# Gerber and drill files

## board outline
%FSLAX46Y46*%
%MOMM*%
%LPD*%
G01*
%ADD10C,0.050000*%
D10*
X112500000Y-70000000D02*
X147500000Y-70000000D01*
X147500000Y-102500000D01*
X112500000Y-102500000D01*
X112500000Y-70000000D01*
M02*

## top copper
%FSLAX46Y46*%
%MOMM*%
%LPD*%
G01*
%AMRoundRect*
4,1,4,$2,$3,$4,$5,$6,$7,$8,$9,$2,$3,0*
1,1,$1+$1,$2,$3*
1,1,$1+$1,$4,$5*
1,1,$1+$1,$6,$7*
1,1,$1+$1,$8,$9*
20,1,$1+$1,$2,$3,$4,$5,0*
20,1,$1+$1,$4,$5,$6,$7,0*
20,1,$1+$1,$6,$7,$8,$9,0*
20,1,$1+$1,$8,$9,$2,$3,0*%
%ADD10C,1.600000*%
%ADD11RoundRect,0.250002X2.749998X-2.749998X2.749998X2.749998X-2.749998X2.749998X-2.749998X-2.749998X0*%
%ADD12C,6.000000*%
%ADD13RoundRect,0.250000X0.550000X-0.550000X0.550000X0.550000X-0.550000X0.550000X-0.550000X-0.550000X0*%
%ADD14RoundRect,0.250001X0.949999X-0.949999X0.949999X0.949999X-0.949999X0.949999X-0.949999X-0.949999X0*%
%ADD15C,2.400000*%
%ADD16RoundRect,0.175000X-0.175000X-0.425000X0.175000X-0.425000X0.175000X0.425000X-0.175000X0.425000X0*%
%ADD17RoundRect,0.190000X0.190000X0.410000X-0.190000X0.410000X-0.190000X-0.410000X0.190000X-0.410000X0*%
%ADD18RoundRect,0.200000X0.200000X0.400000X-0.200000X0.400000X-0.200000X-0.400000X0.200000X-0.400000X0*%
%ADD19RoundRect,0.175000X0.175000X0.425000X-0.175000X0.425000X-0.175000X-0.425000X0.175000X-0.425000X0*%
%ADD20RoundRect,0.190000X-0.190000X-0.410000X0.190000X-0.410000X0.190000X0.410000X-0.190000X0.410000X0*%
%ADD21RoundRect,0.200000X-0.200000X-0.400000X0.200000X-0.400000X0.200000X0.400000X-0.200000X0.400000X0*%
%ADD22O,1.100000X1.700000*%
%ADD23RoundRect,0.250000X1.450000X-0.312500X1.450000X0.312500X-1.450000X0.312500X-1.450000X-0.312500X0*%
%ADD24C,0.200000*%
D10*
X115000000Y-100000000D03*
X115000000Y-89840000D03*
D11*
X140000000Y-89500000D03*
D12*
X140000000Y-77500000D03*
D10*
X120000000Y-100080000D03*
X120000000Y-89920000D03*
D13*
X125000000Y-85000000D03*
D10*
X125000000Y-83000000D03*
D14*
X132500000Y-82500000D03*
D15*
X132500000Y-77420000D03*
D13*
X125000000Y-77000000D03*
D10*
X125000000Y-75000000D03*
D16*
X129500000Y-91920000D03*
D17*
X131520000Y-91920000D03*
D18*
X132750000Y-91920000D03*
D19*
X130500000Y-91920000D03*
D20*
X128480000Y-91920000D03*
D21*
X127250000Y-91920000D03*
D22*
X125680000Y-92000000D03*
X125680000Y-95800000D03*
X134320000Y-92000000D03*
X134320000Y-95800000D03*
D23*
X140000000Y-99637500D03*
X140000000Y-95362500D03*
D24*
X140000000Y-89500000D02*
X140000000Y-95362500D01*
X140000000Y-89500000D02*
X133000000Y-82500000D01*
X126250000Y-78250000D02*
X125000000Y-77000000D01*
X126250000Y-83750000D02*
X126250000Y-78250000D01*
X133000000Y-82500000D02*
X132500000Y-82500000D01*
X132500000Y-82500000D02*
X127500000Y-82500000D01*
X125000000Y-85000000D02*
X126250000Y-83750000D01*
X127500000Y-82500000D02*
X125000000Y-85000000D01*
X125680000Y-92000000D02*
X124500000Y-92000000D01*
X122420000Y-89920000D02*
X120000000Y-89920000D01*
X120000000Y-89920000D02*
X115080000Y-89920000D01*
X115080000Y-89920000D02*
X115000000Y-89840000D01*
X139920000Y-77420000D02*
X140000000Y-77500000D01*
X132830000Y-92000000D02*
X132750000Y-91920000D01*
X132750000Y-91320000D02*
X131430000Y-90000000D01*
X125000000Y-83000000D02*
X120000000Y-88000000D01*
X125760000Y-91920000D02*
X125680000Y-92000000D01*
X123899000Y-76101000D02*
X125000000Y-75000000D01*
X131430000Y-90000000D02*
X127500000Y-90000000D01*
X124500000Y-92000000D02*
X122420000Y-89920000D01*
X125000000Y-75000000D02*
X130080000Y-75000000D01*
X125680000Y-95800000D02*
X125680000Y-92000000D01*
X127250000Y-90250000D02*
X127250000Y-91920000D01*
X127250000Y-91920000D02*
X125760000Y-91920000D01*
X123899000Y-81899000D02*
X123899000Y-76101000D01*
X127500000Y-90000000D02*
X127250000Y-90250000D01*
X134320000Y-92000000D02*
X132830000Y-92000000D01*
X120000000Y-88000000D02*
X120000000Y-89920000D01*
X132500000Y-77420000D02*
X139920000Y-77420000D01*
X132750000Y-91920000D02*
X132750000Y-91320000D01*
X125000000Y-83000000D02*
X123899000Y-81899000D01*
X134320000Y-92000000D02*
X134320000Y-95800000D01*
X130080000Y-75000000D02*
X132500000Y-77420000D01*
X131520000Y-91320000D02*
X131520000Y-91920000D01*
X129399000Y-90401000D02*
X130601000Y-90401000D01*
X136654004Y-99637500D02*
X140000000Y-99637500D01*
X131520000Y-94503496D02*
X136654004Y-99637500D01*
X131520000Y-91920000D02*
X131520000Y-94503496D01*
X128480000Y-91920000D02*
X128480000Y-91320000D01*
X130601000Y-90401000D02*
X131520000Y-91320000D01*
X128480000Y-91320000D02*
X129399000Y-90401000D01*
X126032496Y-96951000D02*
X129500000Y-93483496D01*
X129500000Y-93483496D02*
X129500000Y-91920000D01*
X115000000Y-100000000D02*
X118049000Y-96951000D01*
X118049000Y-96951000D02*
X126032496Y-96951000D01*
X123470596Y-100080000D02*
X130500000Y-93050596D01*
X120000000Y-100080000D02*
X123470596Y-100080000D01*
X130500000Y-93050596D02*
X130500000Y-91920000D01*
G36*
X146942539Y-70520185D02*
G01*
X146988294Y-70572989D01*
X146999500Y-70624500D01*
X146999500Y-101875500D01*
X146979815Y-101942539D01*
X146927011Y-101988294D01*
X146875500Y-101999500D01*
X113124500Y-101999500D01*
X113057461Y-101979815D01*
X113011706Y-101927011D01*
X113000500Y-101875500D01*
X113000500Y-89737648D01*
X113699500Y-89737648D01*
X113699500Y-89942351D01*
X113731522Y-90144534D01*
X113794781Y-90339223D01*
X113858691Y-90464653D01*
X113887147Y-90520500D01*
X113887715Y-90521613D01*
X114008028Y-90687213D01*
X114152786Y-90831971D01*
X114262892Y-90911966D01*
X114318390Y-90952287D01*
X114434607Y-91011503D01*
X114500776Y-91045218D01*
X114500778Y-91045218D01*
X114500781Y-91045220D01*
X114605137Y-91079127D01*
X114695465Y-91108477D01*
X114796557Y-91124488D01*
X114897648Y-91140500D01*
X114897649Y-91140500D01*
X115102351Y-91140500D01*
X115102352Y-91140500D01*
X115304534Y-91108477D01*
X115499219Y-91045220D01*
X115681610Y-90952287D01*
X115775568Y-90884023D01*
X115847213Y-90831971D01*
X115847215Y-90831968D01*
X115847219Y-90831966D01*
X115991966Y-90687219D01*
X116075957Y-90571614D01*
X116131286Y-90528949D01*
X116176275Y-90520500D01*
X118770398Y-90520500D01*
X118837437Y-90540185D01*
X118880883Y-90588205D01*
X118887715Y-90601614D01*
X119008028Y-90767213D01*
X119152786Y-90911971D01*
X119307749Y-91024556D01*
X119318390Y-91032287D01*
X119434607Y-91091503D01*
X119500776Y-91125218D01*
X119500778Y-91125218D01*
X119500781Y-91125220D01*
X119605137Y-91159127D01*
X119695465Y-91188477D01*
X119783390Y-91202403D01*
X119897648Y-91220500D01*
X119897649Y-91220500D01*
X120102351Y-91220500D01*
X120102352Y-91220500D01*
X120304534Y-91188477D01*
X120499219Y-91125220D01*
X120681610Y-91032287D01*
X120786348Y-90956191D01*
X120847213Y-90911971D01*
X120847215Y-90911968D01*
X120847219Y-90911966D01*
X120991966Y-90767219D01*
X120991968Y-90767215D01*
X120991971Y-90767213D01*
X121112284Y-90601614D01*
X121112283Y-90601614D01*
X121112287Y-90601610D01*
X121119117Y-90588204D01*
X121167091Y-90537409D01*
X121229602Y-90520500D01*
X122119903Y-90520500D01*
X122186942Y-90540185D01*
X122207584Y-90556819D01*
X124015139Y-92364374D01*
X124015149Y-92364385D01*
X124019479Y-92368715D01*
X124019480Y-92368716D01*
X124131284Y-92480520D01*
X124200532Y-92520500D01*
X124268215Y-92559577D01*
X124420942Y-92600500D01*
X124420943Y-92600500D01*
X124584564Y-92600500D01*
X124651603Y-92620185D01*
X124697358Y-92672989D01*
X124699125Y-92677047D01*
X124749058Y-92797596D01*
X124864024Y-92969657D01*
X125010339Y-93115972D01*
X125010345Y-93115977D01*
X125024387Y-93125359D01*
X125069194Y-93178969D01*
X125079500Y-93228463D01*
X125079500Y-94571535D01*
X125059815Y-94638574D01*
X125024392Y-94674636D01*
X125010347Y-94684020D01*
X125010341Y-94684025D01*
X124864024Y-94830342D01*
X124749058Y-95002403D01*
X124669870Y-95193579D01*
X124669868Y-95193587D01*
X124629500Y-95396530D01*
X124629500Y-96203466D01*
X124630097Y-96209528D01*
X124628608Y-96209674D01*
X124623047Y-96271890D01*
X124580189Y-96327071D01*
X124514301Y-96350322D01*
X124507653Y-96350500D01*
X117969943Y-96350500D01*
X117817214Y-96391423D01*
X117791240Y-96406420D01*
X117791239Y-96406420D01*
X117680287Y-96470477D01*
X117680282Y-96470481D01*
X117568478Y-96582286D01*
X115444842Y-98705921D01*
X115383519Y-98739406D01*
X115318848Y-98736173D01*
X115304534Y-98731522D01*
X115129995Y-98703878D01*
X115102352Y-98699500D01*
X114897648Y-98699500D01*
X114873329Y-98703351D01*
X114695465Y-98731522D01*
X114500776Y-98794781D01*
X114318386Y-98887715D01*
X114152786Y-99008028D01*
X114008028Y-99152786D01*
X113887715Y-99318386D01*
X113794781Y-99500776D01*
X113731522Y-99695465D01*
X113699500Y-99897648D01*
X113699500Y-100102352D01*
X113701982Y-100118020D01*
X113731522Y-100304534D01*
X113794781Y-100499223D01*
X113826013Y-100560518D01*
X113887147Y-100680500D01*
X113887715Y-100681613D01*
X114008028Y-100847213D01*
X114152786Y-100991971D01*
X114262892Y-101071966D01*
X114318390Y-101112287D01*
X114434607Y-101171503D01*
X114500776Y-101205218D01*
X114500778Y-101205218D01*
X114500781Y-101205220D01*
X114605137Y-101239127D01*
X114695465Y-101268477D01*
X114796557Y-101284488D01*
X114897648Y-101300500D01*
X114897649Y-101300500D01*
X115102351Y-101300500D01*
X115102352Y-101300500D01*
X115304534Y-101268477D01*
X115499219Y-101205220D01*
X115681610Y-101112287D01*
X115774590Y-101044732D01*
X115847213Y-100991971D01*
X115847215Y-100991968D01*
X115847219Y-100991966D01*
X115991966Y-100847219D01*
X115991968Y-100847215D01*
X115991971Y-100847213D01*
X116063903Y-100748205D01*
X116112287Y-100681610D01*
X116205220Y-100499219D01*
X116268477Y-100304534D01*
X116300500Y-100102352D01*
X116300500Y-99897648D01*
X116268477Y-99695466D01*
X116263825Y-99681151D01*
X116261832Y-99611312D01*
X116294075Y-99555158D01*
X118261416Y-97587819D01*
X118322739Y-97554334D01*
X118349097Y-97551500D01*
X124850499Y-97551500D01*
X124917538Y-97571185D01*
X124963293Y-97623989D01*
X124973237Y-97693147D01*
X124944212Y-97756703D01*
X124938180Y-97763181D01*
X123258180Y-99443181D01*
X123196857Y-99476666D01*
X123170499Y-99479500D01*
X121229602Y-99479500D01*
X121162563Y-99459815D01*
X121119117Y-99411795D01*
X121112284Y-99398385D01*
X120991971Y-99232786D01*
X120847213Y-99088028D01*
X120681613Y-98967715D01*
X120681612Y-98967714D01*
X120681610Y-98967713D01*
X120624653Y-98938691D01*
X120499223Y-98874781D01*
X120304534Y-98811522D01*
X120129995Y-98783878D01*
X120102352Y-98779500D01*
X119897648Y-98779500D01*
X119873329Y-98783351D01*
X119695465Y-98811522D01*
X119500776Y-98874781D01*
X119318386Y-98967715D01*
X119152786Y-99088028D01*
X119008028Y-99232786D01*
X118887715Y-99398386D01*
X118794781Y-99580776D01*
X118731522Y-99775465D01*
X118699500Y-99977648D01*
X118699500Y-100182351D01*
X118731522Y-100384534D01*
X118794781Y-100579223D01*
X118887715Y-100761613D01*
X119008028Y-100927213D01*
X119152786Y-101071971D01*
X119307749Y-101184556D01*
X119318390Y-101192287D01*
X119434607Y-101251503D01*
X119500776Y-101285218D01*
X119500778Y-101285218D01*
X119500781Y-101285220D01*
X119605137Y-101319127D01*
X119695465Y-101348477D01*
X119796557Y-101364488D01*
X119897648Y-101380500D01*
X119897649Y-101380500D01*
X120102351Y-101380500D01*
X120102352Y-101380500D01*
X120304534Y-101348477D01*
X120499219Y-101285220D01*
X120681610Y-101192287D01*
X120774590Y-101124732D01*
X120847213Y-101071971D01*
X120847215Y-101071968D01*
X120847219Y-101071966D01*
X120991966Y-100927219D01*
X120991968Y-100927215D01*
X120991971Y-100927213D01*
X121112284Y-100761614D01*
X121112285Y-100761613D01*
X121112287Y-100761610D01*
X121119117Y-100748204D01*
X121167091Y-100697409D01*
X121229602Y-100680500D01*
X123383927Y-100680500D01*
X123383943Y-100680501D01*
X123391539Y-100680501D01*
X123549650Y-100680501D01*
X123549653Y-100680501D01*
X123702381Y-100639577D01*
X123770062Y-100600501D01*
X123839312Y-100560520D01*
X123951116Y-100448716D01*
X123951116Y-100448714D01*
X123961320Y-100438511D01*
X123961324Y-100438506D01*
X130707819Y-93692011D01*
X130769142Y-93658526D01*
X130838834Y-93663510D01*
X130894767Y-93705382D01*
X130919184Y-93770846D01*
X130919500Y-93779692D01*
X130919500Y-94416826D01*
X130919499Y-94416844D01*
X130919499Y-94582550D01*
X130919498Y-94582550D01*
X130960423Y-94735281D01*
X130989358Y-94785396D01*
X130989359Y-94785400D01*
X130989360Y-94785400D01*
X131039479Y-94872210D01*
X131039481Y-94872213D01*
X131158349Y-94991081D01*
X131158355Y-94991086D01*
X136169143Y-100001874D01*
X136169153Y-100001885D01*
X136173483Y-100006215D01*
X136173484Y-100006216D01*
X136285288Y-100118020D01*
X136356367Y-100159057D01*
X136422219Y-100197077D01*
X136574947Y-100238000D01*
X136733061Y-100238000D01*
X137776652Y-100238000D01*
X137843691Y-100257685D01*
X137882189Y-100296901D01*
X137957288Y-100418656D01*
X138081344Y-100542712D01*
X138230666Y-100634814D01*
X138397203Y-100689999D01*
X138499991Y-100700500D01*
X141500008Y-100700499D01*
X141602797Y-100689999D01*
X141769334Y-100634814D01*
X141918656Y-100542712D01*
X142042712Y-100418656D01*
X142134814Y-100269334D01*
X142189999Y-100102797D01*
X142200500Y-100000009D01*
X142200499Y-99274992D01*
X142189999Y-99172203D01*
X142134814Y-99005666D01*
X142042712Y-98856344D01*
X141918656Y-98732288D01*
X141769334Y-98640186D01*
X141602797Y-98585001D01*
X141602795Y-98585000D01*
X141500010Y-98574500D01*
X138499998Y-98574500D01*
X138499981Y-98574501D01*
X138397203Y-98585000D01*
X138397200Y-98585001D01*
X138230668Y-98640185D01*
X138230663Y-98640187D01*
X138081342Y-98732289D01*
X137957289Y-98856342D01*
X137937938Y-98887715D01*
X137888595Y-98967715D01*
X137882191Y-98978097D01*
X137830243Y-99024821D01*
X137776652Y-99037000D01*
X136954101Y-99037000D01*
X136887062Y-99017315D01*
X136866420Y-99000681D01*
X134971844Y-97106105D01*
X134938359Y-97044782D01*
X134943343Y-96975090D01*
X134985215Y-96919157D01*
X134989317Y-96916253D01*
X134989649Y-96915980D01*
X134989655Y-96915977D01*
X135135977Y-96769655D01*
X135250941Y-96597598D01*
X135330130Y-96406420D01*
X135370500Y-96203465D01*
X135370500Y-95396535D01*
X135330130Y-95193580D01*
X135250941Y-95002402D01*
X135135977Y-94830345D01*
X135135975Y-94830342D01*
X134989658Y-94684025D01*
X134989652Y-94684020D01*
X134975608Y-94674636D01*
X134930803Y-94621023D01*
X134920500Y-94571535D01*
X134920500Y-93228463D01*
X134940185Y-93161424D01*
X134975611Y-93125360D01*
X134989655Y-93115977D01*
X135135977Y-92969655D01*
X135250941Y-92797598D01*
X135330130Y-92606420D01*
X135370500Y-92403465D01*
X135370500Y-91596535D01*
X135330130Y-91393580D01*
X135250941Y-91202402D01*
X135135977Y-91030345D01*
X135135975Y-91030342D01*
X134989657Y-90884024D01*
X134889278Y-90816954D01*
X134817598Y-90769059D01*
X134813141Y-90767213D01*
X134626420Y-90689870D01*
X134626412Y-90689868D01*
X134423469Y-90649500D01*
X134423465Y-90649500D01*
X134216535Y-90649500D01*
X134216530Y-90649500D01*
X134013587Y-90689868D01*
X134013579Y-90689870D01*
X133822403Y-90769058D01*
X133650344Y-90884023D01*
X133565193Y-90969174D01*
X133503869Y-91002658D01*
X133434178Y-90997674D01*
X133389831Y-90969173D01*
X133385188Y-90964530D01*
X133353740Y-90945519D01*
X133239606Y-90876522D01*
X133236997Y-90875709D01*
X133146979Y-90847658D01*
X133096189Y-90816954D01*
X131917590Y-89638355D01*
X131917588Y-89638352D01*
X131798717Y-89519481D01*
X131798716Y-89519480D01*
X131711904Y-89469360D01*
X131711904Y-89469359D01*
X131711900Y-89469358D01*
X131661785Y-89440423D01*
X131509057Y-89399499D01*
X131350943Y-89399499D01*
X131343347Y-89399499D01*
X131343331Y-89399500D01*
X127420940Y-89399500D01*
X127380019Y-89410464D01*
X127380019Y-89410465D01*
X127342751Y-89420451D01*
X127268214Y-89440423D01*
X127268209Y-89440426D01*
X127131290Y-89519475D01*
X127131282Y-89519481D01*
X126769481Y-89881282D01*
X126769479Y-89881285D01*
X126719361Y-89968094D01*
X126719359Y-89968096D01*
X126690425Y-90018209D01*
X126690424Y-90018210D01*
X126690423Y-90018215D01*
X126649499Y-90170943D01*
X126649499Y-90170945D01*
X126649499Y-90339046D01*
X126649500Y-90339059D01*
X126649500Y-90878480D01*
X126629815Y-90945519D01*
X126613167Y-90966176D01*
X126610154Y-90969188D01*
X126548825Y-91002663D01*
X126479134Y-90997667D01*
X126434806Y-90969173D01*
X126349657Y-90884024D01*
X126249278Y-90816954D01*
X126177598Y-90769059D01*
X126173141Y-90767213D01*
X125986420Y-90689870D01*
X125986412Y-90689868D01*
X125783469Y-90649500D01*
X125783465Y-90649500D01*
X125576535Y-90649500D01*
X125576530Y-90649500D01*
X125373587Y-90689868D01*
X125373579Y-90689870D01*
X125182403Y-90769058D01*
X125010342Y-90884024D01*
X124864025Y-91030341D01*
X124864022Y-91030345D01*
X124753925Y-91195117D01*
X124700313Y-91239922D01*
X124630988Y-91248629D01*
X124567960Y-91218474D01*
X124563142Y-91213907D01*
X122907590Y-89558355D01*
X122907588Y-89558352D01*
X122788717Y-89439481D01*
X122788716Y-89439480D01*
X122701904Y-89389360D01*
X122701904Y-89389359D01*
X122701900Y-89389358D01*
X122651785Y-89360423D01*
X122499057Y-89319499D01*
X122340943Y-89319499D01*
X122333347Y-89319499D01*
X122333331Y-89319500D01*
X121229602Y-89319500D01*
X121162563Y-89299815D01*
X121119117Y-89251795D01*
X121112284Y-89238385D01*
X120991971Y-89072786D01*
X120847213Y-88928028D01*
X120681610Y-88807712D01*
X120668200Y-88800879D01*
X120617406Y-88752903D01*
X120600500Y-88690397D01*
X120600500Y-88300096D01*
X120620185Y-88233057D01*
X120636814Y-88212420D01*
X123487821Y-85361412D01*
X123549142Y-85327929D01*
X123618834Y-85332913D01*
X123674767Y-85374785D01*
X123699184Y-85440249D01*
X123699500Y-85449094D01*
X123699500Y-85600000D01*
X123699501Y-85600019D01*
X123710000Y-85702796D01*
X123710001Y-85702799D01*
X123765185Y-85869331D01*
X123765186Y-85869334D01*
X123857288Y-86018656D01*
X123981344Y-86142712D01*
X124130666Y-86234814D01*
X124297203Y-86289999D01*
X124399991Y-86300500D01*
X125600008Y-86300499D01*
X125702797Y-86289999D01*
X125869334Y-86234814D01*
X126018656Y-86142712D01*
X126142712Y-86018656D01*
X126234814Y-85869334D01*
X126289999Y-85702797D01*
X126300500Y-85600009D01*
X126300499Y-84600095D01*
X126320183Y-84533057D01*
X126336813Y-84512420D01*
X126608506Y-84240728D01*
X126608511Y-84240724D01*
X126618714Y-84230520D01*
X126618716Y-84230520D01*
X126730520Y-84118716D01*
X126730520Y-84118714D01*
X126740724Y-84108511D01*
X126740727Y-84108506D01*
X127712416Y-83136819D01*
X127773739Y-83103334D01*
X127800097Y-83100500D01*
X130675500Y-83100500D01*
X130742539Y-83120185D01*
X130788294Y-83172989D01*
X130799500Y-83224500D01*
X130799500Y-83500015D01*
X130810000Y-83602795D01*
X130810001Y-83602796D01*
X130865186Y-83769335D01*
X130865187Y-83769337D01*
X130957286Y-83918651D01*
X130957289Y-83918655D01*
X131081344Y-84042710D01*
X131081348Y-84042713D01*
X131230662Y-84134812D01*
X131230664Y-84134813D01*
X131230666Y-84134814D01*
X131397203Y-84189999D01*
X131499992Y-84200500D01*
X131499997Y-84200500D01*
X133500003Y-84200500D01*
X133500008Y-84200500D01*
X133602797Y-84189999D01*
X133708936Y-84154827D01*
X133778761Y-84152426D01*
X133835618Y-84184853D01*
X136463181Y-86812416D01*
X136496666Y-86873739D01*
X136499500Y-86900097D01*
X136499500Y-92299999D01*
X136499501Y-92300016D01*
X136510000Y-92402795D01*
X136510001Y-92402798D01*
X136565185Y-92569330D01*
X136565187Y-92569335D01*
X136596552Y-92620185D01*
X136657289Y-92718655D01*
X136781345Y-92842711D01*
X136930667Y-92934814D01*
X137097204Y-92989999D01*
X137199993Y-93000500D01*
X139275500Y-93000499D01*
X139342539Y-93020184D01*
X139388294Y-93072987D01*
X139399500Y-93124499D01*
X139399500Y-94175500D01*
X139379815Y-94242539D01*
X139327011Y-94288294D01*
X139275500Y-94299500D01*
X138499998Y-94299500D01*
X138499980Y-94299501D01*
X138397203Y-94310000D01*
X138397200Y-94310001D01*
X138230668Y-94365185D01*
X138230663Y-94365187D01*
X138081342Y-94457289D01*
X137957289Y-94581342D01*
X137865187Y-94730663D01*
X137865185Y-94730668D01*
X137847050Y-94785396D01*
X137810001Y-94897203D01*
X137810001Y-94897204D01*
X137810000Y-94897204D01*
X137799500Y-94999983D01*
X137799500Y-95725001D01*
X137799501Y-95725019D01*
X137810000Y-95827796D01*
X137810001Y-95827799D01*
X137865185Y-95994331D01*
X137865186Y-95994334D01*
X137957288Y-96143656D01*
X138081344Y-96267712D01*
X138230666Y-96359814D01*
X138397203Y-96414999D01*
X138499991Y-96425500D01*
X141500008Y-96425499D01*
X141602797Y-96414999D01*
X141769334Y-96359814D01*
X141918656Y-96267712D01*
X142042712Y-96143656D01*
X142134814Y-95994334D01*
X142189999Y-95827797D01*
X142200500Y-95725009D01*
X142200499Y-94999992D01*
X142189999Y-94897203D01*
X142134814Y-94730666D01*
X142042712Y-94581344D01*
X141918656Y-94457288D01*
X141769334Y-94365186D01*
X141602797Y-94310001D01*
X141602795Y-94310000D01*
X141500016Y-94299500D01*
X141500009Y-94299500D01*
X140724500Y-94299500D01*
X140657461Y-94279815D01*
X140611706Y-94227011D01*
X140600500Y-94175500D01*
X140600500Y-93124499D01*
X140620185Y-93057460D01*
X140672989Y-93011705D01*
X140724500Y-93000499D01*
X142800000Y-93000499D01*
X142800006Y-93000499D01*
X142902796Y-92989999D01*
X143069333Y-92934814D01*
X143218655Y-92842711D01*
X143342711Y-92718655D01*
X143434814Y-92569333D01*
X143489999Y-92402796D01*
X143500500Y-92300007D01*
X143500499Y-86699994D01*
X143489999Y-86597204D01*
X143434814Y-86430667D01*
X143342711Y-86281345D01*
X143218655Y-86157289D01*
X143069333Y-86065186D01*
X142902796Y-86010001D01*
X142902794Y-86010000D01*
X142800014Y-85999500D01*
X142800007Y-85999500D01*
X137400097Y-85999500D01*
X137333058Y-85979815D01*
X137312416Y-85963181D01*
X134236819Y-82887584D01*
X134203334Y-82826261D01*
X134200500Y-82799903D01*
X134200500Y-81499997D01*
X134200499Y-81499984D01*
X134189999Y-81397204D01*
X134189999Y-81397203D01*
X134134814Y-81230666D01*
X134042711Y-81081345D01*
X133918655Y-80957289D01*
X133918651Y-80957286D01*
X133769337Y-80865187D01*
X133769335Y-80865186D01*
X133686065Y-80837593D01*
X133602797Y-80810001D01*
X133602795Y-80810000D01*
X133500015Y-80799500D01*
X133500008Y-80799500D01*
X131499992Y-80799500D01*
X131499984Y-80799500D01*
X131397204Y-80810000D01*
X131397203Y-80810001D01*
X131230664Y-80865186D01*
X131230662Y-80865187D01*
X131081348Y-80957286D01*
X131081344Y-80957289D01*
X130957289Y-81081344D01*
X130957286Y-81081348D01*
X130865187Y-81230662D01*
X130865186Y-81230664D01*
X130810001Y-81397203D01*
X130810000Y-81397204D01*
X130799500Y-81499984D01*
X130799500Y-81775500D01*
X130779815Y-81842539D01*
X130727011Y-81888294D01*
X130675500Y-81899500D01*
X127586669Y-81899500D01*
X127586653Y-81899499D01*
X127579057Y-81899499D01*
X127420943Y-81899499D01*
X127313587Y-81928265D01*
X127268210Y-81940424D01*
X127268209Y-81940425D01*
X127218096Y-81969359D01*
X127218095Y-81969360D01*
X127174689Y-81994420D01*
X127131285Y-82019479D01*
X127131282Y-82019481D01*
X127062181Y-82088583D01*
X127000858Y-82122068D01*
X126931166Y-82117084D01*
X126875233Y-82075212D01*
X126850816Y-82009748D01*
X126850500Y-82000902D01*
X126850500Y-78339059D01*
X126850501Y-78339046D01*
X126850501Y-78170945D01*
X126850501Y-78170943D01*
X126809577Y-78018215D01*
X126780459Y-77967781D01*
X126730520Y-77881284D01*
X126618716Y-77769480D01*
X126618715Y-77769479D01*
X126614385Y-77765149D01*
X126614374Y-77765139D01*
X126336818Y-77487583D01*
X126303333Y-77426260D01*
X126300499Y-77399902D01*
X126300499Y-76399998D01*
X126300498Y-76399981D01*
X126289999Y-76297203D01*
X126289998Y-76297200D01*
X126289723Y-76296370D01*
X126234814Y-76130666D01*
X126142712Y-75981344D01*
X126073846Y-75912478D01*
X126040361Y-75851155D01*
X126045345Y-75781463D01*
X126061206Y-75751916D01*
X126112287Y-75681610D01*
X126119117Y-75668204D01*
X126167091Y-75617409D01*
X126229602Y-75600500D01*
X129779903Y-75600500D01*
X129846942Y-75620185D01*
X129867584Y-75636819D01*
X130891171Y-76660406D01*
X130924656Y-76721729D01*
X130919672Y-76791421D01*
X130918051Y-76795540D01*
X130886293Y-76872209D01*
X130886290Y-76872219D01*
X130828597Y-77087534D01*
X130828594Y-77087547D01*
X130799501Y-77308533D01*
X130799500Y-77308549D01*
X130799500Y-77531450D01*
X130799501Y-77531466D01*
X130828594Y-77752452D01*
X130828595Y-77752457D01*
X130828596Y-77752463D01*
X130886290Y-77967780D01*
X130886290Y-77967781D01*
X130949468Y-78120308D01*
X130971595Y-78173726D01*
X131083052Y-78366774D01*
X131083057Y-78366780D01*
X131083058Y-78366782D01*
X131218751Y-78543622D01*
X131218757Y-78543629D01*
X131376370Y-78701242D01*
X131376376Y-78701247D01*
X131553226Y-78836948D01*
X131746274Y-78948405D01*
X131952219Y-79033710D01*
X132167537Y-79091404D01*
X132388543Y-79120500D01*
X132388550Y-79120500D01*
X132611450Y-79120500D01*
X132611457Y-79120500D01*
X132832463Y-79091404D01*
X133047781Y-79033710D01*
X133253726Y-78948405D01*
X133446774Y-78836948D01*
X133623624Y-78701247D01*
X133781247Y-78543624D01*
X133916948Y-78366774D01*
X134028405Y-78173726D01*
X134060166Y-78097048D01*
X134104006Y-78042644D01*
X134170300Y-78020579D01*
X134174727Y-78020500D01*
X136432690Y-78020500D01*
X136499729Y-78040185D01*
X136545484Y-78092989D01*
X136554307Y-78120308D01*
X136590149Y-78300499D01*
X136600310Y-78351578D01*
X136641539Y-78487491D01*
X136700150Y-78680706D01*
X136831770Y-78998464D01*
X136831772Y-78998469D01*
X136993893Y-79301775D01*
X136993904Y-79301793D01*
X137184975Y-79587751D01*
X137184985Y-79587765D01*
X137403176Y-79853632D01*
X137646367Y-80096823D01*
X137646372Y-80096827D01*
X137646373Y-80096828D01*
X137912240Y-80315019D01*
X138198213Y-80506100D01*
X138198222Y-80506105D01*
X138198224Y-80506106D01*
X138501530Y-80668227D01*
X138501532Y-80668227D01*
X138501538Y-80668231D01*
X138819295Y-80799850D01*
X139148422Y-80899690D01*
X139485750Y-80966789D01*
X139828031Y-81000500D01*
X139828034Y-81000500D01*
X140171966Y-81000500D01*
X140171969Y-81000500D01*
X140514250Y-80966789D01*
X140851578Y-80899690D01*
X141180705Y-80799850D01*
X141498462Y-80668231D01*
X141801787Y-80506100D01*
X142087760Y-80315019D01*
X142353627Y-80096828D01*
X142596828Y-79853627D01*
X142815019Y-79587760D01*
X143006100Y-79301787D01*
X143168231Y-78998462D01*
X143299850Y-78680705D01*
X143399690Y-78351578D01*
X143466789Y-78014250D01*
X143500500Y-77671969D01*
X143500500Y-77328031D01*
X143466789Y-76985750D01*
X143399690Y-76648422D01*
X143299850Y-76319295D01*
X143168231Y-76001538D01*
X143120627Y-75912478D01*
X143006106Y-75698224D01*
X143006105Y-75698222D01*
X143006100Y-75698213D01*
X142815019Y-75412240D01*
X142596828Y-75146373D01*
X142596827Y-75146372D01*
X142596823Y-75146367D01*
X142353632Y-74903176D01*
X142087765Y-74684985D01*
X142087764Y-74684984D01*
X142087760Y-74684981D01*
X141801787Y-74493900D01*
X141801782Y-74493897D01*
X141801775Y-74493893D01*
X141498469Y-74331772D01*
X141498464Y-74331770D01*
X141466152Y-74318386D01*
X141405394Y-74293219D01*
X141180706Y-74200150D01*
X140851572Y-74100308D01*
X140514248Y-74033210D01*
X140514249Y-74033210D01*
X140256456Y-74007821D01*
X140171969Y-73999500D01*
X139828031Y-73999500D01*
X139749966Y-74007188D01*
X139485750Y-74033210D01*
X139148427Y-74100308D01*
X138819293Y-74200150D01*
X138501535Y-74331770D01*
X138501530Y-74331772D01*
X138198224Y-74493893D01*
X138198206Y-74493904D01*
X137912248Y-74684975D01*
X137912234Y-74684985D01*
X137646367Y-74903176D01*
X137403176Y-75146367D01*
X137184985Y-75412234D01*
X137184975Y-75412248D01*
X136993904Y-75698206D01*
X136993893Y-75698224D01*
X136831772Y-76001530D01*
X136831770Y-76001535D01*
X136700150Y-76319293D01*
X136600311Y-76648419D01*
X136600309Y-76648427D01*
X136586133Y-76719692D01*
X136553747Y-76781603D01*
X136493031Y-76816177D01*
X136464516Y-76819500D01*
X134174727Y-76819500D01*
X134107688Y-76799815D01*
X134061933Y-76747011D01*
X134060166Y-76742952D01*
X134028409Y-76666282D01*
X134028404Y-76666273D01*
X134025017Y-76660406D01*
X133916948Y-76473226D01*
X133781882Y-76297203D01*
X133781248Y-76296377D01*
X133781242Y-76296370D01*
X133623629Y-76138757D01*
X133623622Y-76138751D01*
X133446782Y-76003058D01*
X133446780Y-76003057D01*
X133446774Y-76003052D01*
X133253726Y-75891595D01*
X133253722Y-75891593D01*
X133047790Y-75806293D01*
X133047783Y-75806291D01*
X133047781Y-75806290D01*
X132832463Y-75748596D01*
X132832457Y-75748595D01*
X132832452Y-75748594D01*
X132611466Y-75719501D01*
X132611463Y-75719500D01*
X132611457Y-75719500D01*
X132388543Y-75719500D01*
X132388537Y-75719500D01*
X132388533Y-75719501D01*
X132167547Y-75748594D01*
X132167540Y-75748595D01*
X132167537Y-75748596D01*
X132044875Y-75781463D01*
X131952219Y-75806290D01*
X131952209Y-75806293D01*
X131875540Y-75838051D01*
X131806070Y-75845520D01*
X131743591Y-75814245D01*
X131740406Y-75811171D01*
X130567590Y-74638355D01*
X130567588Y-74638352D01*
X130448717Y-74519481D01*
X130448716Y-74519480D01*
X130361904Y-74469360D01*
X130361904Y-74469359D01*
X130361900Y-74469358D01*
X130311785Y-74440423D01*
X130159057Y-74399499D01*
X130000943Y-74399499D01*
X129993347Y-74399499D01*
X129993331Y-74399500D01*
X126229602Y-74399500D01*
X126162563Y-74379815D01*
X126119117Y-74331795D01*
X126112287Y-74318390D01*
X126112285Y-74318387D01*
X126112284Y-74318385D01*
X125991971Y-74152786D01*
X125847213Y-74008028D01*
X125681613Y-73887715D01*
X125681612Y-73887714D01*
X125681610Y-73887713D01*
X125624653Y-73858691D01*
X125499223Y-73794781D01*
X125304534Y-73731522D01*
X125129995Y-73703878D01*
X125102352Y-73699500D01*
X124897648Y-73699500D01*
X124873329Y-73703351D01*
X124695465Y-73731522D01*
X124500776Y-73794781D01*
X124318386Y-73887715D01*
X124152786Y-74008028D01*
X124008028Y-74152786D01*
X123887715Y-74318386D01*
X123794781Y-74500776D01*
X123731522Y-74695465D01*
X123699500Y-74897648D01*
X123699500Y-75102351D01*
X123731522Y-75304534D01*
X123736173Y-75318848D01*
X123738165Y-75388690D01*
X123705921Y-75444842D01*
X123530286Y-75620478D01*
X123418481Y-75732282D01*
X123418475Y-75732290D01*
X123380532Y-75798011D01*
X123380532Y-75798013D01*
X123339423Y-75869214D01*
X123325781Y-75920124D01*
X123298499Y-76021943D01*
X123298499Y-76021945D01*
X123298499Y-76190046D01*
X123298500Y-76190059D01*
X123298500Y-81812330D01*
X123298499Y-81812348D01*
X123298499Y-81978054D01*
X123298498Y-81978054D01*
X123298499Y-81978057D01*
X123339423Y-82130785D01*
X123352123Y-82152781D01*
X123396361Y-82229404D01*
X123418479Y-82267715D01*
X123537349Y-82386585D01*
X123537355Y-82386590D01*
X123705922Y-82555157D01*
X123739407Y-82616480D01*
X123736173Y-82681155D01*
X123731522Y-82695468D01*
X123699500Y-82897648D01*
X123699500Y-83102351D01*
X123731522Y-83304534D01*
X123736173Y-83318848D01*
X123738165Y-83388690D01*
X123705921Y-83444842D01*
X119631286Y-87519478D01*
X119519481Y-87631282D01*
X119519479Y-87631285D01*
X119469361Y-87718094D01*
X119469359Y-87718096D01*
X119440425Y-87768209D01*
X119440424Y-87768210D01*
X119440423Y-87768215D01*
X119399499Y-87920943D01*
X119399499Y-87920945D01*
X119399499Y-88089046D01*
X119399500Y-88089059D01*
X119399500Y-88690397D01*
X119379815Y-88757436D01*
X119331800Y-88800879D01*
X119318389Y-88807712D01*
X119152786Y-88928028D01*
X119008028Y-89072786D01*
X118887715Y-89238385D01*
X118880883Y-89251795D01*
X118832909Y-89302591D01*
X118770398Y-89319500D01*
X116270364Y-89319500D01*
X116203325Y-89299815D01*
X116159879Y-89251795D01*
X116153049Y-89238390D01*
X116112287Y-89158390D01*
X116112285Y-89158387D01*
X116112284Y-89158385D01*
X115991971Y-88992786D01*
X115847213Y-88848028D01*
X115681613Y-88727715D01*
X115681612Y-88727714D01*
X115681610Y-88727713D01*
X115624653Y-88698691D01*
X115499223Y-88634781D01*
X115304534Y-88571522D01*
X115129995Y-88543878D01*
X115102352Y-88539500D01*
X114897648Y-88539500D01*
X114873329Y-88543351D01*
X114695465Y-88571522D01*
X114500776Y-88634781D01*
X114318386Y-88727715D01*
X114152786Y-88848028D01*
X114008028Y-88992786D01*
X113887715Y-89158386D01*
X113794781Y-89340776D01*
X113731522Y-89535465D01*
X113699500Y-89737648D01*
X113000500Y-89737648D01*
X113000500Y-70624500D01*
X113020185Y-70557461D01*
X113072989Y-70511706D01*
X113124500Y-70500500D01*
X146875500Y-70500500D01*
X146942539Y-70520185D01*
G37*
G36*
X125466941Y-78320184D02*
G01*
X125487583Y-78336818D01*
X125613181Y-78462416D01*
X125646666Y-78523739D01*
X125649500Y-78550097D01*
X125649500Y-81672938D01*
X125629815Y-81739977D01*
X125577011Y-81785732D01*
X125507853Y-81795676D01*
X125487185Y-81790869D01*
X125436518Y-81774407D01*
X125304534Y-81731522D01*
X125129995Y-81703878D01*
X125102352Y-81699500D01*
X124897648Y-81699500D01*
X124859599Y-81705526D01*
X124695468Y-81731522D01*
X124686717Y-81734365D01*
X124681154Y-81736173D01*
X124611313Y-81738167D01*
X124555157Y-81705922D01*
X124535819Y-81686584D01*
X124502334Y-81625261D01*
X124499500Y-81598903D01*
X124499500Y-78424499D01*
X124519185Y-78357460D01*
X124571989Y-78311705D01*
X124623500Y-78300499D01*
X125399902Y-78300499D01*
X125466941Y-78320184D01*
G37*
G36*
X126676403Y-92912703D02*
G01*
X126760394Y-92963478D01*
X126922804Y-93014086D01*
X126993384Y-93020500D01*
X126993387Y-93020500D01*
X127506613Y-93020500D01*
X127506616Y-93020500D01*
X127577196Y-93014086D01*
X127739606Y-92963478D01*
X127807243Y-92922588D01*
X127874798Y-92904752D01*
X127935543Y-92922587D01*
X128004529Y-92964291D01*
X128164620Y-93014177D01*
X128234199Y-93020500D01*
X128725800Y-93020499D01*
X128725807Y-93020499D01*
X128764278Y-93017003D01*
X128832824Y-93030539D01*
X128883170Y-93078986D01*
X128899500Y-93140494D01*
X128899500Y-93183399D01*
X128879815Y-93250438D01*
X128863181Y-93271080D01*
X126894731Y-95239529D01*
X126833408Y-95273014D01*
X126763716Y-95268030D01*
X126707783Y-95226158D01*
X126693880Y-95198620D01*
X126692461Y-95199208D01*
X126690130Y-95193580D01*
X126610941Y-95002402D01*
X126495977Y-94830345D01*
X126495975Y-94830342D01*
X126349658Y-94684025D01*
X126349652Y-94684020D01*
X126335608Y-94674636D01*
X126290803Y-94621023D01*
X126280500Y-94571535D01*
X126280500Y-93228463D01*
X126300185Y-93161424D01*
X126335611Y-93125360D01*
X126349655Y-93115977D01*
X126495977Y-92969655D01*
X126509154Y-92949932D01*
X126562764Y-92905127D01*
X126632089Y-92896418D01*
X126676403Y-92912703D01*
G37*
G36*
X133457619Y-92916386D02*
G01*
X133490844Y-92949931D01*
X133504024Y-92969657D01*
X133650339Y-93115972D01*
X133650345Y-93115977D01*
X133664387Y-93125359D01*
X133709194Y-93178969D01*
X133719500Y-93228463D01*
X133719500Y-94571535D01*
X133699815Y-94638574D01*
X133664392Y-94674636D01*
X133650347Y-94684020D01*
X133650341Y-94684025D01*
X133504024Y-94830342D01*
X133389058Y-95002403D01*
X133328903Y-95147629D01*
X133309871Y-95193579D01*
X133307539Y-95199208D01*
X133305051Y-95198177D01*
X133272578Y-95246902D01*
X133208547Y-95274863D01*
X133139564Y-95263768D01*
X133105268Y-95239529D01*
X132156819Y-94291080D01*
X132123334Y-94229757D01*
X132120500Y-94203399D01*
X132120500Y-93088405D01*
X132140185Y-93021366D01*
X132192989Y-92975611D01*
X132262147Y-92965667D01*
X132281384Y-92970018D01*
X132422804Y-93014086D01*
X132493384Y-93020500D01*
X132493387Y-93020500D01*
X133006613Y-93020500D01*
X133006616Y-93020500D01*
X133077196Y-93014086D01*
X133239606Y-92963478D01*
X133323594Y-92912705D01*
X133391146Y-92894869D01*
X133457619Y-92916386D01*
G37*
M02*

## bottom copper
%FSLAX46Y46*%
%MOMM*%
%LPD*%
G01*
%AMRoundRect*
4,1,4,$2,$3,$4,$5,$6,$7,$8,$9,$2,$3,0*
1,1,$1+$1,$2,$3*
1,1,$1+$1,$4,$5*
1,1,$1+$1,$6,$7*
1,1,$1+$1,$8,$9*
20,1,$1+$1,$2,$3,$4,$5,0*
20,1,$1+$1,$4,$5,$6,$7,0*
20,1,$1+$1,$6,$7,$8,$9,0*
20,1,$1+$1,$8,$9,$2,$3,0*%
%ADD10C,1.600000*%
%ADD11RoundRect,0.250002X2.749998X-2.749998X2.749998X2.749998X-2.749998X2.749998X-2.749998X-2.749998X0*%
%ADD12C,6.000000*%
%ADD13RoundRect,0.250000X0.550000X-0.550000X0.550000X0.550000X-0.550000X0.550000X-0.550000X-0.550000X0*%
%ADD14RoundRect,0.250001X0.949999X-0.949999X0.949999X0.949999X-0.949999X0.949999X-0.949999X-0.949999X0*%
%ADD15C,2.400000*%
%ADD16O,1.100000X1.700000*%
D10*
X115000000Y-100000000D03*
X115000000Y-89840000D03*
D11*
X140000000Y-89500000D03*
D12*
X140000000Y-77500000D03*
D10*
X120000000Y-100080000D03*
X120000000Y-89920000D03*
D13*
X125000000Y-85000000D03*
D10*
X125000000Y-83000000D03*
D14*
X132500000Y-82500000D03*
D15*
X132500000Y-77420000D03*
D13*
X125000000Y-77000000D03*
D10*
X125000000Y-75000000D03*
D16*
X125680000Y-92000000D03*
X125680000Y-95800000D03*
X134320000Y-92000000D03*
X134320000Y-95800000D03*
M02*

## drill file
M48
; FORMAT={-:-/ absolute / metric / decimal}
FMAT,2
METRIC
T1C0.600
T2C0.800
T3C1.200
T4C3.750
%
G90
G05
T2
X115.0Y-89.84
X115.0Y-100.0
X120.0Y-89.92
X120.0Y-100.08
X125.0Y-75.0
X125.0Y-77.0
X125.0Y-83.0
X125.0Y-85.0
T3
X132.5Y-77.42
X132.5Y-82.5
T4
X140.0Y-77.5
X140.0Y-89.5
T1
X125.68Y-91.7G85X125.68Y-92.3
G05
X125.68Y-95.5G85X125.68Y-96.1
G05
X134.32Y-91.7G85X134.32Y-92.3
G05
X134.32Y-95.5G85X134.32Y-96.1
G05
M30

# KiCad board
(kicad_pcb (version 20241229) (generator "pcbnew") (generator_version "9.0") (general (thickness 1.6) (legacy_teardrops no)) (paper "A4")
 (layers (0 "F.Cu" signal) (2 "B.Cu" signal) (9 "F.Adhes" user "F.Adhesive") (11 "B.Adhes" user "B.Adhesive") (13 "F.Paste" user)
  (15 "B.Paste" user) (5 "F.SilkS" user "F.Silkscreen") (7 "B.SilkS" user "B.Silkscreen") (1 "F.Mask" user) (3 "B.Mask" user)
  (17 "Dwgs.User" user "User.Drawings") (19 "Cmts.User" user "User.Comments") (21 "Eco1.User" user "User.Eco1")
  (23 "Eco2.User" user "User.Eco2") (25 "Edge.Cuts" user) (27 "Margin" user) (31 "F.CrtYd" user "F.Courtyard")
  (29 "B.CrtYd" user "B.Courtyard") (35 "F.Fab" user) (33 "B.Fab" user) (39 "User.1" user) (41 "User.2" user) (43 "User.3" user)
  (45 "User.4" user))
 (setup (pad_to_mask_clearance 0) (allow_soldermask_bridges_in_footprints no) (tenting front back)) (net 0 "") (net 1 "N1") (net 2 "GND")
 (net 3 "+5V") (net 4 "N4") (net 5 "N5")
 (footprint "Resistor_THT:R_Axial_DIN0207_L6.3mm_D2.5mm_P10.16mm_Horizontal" (layer "F.Cu") (at 115 100 90)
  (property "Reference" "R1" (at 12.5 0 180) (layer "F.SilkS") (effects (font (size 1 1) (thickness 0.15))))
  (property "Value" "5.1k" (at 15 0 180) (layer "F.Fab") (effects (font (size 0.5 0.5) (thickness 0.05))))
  (pad "1" thru_hole circle (at 0 0 90) (size 1.6 1.6) (drill 0.8) (layers "*.Cu" "*.Mask") (remove_unused_layers no) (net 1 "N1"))
  (pad "2" thru_hole circle (at 10.16 0 90) (size 1.6 1.6) (drill 0.8) (layers "*.Cu" "*.Mask") (remove_unused_layers no) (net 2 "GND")))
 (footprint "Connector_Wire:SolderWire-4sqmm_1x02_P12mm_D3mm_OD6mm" (layer "F.Cu") (at 140 89.5 90)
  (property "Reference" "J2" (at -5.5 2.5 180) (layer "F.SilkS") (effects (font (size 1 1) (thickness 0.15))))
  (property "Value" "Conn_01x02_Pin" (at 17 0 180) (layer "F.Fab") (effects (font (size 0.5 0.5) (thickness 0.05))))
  (pad "1" thru_hole roundrect (at 0 0 90) (size 6 6) (drill 3.75) (layers "*.Cu" "*.Mask") (remove_unused_layers no)
   (roundrect_rratio 0.041667) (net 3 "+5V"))
  (pad "2" thru_hole circle (at 12 0 90) (size 6 6) (drill 3.75) (layers "*.Cu" "*.Mask") (remove_unused_layers no) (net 2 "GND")))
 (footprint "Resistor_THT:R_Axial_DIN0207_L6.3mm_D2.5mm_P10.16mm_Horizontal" (layer "F.Cu") (at 120 100.08 90)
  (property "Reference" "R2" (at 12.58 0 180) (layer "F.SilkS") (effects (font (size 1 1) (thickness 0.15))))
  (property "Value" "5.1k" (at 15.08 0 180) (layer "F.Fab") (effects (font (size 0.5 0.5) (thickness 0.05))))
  (pad "1" thru_hole circle (at 0 0 90) (size 1.6 1.6) (drill 0.8) (layers "*.Cu" "*.Mask") (remove_unused_layers no) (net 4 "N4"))
  (pad "2" thru_hole circle (at 10.16 0 90) (size 1.6 1.6) (drill 0.8) (layers "*.Cu" "*.Mask") (remove_unused_layers no) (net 2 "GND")))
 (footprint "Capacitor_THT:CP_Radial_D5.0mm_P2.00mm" (layer "F.Cu") (at 125 85 90)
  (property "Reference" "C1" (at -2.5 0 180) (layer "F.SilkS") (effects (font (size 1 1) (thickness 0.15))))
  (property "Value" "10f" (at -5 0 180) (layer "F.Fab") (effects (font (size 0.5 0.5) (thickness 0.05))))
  (pad "1" thru_hole roundrect (at 0 0 90) (size 1.6 1.6) (drill 0.8) (layers "*.Cu" "*.Mask") (remove_unused_layers no)
   (roundrect_rratio 0.15625) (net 3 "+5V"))
  (pad "2" thru_hole circle (at 2 0 90) (size 1.6 1.6) (drill 0.8) (layers "*.Cu" "*.Mask") (remove_unused_layers no) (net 2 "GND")))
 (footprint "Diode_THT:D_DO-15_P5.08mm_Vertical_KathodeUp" (layer "F.Cu") (at 132.5 82.5 90)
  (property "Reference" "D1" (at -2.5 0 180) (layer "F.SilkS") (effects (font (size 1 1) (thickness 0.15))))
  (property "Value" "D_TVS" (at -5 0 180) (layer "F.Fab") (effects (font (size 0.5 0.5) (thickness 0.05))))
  (pad "1" thru_hole roundrect (at 0 0 90) (size 2.4 2.4) (drill 1.2) (layers "*.Cu" "*.Mask") (remove_unused_layers no)
   (roundrect_rratio 0.104167) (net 3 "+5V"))
  (pad "2" thru_hole circle (at 5.08 0 90) (size 2.4 2.4) (drill 1.2) (layers "*.Cu" "*.Mask") (remove_unused_layers no) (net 2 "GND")))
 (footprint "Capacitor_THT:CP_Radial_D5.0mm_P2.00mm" (layer "F.Cu") (at 125 77 90)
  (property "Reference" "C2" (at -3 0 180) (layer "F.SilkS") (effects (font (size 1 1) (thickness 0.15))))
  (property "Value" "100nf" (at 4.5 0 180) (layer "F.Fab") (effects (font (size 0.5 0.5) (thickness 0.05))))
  (pad "1" thru_hole roundrect (at 0 0 90) (size 1.6 1.6) (drill 0.8) (layers "*.Cu" "*.Mask") (remove_unused_layers no)
   (roundrect_rratio 0.15625) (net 3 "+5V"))
  (pad "2" thru_hole circle (at 2 0 90) (size 1.6 1.6) (drill 0.8) (layers "*.Cu" "*.Mask") (remove_unused_layers no) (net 2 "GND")))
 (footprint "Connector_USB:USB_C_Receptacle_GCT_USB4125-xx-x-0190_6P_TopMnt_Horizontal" (layer "F.Cu") (at 130 95)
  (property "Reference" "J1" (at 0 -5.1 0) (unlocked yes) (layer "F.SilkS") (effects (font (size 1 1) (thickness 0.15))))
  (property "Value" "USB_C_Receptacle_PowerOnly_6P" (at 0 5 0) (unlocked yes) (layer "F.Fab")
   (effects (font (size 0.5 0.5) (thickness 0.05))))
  (pad "A5" smd roundrect (at -0.5 -3.08) (size 0.7 1.2) (layers "F.Cu" "F.Mask" "F.Paste") (roundrect_rratio 0.25) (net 1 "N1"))
  (pad "A9" smd roundrect (at 1.52 -3.08 180) (size 0.76 1.2) (layers "F.Cu" "F.Mask" "F.Paste") (roundrect_rratio 0.25) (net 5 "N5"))
  (pad "A12" smd roundrect (at 2.75 -3.08 180) (size 0.8 1.2) (layers "F.Cu" "F.Mask" "F.Paste") (roundrect_rratio 0.25) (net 2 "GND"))
  (pad "B5" smd roundrect (at 0.5 -3.08 180) (size 0.7 1.2) (layers "F.Cu" "F.Mask" "F.Paste") (roundrect_rratio 0.25) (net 4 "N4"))
  (pad "B9" smd roundrect (at -1.52 -3.08) (size 0.76 1.2) (layers "F.Cu" "F.Mask" "F.Paste") (roundrect_rratio 0.25) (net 5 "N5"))
  (pad "B12" smd roundrect (at -2.75 -3.08) (size 0.8 1.2) (layers "F.Cu" "F.Mask" "F.Paste") (roundrect_rratio 0.25) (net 2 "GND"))
  (pad "S1" thru_hole oval (at -4.32 -3) (size 1.1 1.7) (drill oval 0.6 1.2) (layers "*.Cu" "*.Mask" "F.Paste") (remove_unused_layers no)
   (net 2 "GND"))
  (pad "S1" thru_hole oval (at -4.32 0.8) (size 1.1 1.7) (drill oval 0.6 1.2) (layers "*.Cu" "*.Mask" "F.Paste") (remove_unused_layers no)
   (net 2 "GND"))
  (pad "S1" thru_hole oval (at 4.32 -3) (size 1.1 1.7) (drill oval 0.6 1.2) (layers "*.Cu" "*.Mask" "F.Paste") (remove_unused_layers no)
   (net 2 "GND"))
  (pad "S1" thru_hole oval (at 4.32 0.8) (size 1.1 1.7) (drill oval 0.6 1.2) (layers "*.Cu" "*.Mask" "F.Paste") (remove_unused_layers no)
   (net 2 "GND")))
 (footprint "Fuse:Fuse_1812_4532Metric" (layer "F.Cu") (at 140 97.5 90)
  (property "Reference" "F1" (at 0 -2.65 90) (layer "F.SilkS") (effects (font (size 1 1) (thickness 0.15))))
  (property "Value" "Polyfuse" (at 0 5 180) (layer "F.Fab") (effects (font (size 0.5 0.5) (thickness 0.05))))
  (pad "1" smd roundrect (at -2.1375 0 90) (size 1.125 3.4) (layers "F.Cu" "F.Mask" "F.Paste") (roundrect_rratio 0.222222) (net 5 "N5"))
  (pad "2" smd roundrect (at 2.1375 0 90) (size 1.125 3.4) (layers "F.Cu" "F.Mask" "F.Paste") (roundrect_rratio 0.222222) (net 3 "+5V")))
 (gr_rect (start 112.5 70) (end 147.5 102.5) (stroke (width 0.05) (type default)) (fill no) (layer "Edge.Cuts"))
 (segment (start 140 89.5) (end 140 95.3625) (width 0.2) (layer "F.Cu") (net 3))
 (segment (start 140 89.5) (end 133 82.5) (width 0.2) (layer "F.Cu") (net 3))
 (segment (start 126.25 78.25) (end 125 77) (width 0.2) (layer "F.Cu") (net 3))
 (segment (start 126.25 83.75) (end 126.25 78.25) (width 0.2) (layer "F.Cu") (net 3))
 (segment (start 133 82.5) (end 132.5 82.5) (width 0.2) (layer "F.Cu") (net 3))
 (segment (start 132.5 82.5) (end 127.5 82.5) (width 0.2) (layer "F.Cu") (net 3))
 (segment (start 125 85) (end 126.25 83.75) (width 0.2) (layer "F.Cu") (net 3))
 (segment (start 127.5 82.5) (end 125 85) (width 0.2) (layer "F.Cu") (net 3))
 (segment (start 125.68 92) (end 124.5 92) (width 0.2) (layer "F.Cu") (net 2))
 (segment (start 122.42 89.92) (end 120 89.92) (width 0.2) (layer "F.Cu") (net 2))
 (segment (start 120 89.92) (end 115.08 89.92) (width 0.2) (layer "F.Cu") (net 2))
 (segment (start 115.08 89.92) (end 115 89.84) (width 0.2) (layer "F.Cu") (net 2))
 (segment (start 139.92 77.42) (end 140 77.5) (width 0.2) (layer "F.Cu") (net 2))
 (segment (start 132.83 92) (end 132.75 91.92) (width 0.2) (layer "F.Cu") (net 2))
 (segment (start 132.75 91.32) (end 131.43 90) (width 0.2) (layer "F.Cu") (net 2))
 (segment (start 125 83) (end 120 88) (width 0.2) (layer "F.Cu") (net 2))
 (segment (start 125.76 91.92) (end 125.68 92) (width 0.2) (layer "F.Cu") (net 2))
 (segment (start 123.899 76.101) (end 125 75) (width 0.2) (layer "F.Cu") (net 2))
 (segment (start 131.43 90) (end 127.5 90) (width 0.2) (layer "F.Cu") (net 2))
 (segment (start 124.5 92) (end 122.42 89.92) (width 0.2) (layer "F.Cu") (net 2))
 (segment (start 125 75) (end 130.08 75) (width 0.2) (layer "F.Cu") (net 2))
 (segment (start 125.68 95.8) (end 125.68 92) (width 0.2) (layer "F.Cu") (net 2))
 (segment (start 127.25 90.25) (end 127.25 91.92) (width 0.2) (layer "F.Cu") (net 2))
 (segment (start 127.25 91.92) (end 125.76 91.92) (width 0.2) (layer "F.Cu") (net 2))
 (segment (start 123.899 81.899) (end 123.899 76.101) (width 0.2) (layer "F.Cu") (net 2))
 (segment (start 127.5 90) (end 127.25 90.25) (width 0.2) (layer "F.Cu") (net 2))
 (segment (start 134.32 92) (end 132.83 92) (width 0.2) (layer "F.Cu") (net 2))
 (segment (start 120 88) (end 120 89.92) (width 0.2) (layer "F.Cu") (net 2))
 (segment (start 132.5 77.42) (end 139.92 77.42) (width 0.2) (layer "F.Cu") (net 2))
 (segment (start 132.75 91.92) (end 132.75 91.32) (width 0.2) (layer "F.Cu") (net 2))
 (segment (start 125 83) (end 123.899 81.899) (width 0.2) (layer "F.Cu") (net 2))
 (segment (start 134.32 92) (end 134.32 95.8) (width 0.2) (layer "F.Cu") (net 2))
 (segment (start 130.08 75) (end 132.5 77.42) (width 0.2) (layer "F.Cu") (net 2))
 (segment (start 131.52 91.32) (end 131.52 91.92) (width 0.2) (layer "F.Cu") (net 5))
 (segment (start 129.399 90.401) (end 130.601 90.401) (width 0.2) (layer "F.Cu") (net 5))
 (segment (start 136.654004 99.6375) (end 140 99.6375) (width 0.2) (layer "F.Cu") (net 5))
 (segment (start 131.52 94.503496) (end 136.654004 99.6375) (width 0.2) (layer "F.Cu") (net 5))
 (segment (start 131.52 91.92) (end 131.52 94.503496) (width 0.2) (layer "F.Cu") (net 5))
 (segment (start 128.48 91.92) (end 128.48 91.32) (width 0.2) (layer "F.Cu") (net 5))
 (segment (start 130.601 90.401) (end 131.52 91.32) (width 0.2) (layer "F.Cu") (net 5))
 (segment (start 128.48 91.32) (end 129.399 90.401) (width 0.2) (layer "F.Cu") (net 5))
 (segment (start 126.032496 96.951) (end 129.5 93.483496) (width 0.2) (layer "F.Cu") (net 1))
 (segment (start 129.5 93.483496) (end 129.5 91.92) (width 0.2) (layer "F.Cu") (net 1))
 (segment (start 115 100) (end 118.049 96.951) (width 0.2) (layer "F.Cu") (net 1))
 (segment (start 118.049 96.951) (end 126.032496 96.951) (width 0.2) (layer "F.Cu") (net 1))
 (segment (start 123.470596 100.08) (end 130.5 93.050596) (width 0.2) (layer "F.Cu") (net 4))
 (segment (start 120 100.08) (end 123.470596 100.08) (width 0.2) (layer "F.Cu") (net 4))
 (segment (start 130.5 93.050596) (end 130.5 91.92) (width 0.2) (layer "F.Cu") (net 4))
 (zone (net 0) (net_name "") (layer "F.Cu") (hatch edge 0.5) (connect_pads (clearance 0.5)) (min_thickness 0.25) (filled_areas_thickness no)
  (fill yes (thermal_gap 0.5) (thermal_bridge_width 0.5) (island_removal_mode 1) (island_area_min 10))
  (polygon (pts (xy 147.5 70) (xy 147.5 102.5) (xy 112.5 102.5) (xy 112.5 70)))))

